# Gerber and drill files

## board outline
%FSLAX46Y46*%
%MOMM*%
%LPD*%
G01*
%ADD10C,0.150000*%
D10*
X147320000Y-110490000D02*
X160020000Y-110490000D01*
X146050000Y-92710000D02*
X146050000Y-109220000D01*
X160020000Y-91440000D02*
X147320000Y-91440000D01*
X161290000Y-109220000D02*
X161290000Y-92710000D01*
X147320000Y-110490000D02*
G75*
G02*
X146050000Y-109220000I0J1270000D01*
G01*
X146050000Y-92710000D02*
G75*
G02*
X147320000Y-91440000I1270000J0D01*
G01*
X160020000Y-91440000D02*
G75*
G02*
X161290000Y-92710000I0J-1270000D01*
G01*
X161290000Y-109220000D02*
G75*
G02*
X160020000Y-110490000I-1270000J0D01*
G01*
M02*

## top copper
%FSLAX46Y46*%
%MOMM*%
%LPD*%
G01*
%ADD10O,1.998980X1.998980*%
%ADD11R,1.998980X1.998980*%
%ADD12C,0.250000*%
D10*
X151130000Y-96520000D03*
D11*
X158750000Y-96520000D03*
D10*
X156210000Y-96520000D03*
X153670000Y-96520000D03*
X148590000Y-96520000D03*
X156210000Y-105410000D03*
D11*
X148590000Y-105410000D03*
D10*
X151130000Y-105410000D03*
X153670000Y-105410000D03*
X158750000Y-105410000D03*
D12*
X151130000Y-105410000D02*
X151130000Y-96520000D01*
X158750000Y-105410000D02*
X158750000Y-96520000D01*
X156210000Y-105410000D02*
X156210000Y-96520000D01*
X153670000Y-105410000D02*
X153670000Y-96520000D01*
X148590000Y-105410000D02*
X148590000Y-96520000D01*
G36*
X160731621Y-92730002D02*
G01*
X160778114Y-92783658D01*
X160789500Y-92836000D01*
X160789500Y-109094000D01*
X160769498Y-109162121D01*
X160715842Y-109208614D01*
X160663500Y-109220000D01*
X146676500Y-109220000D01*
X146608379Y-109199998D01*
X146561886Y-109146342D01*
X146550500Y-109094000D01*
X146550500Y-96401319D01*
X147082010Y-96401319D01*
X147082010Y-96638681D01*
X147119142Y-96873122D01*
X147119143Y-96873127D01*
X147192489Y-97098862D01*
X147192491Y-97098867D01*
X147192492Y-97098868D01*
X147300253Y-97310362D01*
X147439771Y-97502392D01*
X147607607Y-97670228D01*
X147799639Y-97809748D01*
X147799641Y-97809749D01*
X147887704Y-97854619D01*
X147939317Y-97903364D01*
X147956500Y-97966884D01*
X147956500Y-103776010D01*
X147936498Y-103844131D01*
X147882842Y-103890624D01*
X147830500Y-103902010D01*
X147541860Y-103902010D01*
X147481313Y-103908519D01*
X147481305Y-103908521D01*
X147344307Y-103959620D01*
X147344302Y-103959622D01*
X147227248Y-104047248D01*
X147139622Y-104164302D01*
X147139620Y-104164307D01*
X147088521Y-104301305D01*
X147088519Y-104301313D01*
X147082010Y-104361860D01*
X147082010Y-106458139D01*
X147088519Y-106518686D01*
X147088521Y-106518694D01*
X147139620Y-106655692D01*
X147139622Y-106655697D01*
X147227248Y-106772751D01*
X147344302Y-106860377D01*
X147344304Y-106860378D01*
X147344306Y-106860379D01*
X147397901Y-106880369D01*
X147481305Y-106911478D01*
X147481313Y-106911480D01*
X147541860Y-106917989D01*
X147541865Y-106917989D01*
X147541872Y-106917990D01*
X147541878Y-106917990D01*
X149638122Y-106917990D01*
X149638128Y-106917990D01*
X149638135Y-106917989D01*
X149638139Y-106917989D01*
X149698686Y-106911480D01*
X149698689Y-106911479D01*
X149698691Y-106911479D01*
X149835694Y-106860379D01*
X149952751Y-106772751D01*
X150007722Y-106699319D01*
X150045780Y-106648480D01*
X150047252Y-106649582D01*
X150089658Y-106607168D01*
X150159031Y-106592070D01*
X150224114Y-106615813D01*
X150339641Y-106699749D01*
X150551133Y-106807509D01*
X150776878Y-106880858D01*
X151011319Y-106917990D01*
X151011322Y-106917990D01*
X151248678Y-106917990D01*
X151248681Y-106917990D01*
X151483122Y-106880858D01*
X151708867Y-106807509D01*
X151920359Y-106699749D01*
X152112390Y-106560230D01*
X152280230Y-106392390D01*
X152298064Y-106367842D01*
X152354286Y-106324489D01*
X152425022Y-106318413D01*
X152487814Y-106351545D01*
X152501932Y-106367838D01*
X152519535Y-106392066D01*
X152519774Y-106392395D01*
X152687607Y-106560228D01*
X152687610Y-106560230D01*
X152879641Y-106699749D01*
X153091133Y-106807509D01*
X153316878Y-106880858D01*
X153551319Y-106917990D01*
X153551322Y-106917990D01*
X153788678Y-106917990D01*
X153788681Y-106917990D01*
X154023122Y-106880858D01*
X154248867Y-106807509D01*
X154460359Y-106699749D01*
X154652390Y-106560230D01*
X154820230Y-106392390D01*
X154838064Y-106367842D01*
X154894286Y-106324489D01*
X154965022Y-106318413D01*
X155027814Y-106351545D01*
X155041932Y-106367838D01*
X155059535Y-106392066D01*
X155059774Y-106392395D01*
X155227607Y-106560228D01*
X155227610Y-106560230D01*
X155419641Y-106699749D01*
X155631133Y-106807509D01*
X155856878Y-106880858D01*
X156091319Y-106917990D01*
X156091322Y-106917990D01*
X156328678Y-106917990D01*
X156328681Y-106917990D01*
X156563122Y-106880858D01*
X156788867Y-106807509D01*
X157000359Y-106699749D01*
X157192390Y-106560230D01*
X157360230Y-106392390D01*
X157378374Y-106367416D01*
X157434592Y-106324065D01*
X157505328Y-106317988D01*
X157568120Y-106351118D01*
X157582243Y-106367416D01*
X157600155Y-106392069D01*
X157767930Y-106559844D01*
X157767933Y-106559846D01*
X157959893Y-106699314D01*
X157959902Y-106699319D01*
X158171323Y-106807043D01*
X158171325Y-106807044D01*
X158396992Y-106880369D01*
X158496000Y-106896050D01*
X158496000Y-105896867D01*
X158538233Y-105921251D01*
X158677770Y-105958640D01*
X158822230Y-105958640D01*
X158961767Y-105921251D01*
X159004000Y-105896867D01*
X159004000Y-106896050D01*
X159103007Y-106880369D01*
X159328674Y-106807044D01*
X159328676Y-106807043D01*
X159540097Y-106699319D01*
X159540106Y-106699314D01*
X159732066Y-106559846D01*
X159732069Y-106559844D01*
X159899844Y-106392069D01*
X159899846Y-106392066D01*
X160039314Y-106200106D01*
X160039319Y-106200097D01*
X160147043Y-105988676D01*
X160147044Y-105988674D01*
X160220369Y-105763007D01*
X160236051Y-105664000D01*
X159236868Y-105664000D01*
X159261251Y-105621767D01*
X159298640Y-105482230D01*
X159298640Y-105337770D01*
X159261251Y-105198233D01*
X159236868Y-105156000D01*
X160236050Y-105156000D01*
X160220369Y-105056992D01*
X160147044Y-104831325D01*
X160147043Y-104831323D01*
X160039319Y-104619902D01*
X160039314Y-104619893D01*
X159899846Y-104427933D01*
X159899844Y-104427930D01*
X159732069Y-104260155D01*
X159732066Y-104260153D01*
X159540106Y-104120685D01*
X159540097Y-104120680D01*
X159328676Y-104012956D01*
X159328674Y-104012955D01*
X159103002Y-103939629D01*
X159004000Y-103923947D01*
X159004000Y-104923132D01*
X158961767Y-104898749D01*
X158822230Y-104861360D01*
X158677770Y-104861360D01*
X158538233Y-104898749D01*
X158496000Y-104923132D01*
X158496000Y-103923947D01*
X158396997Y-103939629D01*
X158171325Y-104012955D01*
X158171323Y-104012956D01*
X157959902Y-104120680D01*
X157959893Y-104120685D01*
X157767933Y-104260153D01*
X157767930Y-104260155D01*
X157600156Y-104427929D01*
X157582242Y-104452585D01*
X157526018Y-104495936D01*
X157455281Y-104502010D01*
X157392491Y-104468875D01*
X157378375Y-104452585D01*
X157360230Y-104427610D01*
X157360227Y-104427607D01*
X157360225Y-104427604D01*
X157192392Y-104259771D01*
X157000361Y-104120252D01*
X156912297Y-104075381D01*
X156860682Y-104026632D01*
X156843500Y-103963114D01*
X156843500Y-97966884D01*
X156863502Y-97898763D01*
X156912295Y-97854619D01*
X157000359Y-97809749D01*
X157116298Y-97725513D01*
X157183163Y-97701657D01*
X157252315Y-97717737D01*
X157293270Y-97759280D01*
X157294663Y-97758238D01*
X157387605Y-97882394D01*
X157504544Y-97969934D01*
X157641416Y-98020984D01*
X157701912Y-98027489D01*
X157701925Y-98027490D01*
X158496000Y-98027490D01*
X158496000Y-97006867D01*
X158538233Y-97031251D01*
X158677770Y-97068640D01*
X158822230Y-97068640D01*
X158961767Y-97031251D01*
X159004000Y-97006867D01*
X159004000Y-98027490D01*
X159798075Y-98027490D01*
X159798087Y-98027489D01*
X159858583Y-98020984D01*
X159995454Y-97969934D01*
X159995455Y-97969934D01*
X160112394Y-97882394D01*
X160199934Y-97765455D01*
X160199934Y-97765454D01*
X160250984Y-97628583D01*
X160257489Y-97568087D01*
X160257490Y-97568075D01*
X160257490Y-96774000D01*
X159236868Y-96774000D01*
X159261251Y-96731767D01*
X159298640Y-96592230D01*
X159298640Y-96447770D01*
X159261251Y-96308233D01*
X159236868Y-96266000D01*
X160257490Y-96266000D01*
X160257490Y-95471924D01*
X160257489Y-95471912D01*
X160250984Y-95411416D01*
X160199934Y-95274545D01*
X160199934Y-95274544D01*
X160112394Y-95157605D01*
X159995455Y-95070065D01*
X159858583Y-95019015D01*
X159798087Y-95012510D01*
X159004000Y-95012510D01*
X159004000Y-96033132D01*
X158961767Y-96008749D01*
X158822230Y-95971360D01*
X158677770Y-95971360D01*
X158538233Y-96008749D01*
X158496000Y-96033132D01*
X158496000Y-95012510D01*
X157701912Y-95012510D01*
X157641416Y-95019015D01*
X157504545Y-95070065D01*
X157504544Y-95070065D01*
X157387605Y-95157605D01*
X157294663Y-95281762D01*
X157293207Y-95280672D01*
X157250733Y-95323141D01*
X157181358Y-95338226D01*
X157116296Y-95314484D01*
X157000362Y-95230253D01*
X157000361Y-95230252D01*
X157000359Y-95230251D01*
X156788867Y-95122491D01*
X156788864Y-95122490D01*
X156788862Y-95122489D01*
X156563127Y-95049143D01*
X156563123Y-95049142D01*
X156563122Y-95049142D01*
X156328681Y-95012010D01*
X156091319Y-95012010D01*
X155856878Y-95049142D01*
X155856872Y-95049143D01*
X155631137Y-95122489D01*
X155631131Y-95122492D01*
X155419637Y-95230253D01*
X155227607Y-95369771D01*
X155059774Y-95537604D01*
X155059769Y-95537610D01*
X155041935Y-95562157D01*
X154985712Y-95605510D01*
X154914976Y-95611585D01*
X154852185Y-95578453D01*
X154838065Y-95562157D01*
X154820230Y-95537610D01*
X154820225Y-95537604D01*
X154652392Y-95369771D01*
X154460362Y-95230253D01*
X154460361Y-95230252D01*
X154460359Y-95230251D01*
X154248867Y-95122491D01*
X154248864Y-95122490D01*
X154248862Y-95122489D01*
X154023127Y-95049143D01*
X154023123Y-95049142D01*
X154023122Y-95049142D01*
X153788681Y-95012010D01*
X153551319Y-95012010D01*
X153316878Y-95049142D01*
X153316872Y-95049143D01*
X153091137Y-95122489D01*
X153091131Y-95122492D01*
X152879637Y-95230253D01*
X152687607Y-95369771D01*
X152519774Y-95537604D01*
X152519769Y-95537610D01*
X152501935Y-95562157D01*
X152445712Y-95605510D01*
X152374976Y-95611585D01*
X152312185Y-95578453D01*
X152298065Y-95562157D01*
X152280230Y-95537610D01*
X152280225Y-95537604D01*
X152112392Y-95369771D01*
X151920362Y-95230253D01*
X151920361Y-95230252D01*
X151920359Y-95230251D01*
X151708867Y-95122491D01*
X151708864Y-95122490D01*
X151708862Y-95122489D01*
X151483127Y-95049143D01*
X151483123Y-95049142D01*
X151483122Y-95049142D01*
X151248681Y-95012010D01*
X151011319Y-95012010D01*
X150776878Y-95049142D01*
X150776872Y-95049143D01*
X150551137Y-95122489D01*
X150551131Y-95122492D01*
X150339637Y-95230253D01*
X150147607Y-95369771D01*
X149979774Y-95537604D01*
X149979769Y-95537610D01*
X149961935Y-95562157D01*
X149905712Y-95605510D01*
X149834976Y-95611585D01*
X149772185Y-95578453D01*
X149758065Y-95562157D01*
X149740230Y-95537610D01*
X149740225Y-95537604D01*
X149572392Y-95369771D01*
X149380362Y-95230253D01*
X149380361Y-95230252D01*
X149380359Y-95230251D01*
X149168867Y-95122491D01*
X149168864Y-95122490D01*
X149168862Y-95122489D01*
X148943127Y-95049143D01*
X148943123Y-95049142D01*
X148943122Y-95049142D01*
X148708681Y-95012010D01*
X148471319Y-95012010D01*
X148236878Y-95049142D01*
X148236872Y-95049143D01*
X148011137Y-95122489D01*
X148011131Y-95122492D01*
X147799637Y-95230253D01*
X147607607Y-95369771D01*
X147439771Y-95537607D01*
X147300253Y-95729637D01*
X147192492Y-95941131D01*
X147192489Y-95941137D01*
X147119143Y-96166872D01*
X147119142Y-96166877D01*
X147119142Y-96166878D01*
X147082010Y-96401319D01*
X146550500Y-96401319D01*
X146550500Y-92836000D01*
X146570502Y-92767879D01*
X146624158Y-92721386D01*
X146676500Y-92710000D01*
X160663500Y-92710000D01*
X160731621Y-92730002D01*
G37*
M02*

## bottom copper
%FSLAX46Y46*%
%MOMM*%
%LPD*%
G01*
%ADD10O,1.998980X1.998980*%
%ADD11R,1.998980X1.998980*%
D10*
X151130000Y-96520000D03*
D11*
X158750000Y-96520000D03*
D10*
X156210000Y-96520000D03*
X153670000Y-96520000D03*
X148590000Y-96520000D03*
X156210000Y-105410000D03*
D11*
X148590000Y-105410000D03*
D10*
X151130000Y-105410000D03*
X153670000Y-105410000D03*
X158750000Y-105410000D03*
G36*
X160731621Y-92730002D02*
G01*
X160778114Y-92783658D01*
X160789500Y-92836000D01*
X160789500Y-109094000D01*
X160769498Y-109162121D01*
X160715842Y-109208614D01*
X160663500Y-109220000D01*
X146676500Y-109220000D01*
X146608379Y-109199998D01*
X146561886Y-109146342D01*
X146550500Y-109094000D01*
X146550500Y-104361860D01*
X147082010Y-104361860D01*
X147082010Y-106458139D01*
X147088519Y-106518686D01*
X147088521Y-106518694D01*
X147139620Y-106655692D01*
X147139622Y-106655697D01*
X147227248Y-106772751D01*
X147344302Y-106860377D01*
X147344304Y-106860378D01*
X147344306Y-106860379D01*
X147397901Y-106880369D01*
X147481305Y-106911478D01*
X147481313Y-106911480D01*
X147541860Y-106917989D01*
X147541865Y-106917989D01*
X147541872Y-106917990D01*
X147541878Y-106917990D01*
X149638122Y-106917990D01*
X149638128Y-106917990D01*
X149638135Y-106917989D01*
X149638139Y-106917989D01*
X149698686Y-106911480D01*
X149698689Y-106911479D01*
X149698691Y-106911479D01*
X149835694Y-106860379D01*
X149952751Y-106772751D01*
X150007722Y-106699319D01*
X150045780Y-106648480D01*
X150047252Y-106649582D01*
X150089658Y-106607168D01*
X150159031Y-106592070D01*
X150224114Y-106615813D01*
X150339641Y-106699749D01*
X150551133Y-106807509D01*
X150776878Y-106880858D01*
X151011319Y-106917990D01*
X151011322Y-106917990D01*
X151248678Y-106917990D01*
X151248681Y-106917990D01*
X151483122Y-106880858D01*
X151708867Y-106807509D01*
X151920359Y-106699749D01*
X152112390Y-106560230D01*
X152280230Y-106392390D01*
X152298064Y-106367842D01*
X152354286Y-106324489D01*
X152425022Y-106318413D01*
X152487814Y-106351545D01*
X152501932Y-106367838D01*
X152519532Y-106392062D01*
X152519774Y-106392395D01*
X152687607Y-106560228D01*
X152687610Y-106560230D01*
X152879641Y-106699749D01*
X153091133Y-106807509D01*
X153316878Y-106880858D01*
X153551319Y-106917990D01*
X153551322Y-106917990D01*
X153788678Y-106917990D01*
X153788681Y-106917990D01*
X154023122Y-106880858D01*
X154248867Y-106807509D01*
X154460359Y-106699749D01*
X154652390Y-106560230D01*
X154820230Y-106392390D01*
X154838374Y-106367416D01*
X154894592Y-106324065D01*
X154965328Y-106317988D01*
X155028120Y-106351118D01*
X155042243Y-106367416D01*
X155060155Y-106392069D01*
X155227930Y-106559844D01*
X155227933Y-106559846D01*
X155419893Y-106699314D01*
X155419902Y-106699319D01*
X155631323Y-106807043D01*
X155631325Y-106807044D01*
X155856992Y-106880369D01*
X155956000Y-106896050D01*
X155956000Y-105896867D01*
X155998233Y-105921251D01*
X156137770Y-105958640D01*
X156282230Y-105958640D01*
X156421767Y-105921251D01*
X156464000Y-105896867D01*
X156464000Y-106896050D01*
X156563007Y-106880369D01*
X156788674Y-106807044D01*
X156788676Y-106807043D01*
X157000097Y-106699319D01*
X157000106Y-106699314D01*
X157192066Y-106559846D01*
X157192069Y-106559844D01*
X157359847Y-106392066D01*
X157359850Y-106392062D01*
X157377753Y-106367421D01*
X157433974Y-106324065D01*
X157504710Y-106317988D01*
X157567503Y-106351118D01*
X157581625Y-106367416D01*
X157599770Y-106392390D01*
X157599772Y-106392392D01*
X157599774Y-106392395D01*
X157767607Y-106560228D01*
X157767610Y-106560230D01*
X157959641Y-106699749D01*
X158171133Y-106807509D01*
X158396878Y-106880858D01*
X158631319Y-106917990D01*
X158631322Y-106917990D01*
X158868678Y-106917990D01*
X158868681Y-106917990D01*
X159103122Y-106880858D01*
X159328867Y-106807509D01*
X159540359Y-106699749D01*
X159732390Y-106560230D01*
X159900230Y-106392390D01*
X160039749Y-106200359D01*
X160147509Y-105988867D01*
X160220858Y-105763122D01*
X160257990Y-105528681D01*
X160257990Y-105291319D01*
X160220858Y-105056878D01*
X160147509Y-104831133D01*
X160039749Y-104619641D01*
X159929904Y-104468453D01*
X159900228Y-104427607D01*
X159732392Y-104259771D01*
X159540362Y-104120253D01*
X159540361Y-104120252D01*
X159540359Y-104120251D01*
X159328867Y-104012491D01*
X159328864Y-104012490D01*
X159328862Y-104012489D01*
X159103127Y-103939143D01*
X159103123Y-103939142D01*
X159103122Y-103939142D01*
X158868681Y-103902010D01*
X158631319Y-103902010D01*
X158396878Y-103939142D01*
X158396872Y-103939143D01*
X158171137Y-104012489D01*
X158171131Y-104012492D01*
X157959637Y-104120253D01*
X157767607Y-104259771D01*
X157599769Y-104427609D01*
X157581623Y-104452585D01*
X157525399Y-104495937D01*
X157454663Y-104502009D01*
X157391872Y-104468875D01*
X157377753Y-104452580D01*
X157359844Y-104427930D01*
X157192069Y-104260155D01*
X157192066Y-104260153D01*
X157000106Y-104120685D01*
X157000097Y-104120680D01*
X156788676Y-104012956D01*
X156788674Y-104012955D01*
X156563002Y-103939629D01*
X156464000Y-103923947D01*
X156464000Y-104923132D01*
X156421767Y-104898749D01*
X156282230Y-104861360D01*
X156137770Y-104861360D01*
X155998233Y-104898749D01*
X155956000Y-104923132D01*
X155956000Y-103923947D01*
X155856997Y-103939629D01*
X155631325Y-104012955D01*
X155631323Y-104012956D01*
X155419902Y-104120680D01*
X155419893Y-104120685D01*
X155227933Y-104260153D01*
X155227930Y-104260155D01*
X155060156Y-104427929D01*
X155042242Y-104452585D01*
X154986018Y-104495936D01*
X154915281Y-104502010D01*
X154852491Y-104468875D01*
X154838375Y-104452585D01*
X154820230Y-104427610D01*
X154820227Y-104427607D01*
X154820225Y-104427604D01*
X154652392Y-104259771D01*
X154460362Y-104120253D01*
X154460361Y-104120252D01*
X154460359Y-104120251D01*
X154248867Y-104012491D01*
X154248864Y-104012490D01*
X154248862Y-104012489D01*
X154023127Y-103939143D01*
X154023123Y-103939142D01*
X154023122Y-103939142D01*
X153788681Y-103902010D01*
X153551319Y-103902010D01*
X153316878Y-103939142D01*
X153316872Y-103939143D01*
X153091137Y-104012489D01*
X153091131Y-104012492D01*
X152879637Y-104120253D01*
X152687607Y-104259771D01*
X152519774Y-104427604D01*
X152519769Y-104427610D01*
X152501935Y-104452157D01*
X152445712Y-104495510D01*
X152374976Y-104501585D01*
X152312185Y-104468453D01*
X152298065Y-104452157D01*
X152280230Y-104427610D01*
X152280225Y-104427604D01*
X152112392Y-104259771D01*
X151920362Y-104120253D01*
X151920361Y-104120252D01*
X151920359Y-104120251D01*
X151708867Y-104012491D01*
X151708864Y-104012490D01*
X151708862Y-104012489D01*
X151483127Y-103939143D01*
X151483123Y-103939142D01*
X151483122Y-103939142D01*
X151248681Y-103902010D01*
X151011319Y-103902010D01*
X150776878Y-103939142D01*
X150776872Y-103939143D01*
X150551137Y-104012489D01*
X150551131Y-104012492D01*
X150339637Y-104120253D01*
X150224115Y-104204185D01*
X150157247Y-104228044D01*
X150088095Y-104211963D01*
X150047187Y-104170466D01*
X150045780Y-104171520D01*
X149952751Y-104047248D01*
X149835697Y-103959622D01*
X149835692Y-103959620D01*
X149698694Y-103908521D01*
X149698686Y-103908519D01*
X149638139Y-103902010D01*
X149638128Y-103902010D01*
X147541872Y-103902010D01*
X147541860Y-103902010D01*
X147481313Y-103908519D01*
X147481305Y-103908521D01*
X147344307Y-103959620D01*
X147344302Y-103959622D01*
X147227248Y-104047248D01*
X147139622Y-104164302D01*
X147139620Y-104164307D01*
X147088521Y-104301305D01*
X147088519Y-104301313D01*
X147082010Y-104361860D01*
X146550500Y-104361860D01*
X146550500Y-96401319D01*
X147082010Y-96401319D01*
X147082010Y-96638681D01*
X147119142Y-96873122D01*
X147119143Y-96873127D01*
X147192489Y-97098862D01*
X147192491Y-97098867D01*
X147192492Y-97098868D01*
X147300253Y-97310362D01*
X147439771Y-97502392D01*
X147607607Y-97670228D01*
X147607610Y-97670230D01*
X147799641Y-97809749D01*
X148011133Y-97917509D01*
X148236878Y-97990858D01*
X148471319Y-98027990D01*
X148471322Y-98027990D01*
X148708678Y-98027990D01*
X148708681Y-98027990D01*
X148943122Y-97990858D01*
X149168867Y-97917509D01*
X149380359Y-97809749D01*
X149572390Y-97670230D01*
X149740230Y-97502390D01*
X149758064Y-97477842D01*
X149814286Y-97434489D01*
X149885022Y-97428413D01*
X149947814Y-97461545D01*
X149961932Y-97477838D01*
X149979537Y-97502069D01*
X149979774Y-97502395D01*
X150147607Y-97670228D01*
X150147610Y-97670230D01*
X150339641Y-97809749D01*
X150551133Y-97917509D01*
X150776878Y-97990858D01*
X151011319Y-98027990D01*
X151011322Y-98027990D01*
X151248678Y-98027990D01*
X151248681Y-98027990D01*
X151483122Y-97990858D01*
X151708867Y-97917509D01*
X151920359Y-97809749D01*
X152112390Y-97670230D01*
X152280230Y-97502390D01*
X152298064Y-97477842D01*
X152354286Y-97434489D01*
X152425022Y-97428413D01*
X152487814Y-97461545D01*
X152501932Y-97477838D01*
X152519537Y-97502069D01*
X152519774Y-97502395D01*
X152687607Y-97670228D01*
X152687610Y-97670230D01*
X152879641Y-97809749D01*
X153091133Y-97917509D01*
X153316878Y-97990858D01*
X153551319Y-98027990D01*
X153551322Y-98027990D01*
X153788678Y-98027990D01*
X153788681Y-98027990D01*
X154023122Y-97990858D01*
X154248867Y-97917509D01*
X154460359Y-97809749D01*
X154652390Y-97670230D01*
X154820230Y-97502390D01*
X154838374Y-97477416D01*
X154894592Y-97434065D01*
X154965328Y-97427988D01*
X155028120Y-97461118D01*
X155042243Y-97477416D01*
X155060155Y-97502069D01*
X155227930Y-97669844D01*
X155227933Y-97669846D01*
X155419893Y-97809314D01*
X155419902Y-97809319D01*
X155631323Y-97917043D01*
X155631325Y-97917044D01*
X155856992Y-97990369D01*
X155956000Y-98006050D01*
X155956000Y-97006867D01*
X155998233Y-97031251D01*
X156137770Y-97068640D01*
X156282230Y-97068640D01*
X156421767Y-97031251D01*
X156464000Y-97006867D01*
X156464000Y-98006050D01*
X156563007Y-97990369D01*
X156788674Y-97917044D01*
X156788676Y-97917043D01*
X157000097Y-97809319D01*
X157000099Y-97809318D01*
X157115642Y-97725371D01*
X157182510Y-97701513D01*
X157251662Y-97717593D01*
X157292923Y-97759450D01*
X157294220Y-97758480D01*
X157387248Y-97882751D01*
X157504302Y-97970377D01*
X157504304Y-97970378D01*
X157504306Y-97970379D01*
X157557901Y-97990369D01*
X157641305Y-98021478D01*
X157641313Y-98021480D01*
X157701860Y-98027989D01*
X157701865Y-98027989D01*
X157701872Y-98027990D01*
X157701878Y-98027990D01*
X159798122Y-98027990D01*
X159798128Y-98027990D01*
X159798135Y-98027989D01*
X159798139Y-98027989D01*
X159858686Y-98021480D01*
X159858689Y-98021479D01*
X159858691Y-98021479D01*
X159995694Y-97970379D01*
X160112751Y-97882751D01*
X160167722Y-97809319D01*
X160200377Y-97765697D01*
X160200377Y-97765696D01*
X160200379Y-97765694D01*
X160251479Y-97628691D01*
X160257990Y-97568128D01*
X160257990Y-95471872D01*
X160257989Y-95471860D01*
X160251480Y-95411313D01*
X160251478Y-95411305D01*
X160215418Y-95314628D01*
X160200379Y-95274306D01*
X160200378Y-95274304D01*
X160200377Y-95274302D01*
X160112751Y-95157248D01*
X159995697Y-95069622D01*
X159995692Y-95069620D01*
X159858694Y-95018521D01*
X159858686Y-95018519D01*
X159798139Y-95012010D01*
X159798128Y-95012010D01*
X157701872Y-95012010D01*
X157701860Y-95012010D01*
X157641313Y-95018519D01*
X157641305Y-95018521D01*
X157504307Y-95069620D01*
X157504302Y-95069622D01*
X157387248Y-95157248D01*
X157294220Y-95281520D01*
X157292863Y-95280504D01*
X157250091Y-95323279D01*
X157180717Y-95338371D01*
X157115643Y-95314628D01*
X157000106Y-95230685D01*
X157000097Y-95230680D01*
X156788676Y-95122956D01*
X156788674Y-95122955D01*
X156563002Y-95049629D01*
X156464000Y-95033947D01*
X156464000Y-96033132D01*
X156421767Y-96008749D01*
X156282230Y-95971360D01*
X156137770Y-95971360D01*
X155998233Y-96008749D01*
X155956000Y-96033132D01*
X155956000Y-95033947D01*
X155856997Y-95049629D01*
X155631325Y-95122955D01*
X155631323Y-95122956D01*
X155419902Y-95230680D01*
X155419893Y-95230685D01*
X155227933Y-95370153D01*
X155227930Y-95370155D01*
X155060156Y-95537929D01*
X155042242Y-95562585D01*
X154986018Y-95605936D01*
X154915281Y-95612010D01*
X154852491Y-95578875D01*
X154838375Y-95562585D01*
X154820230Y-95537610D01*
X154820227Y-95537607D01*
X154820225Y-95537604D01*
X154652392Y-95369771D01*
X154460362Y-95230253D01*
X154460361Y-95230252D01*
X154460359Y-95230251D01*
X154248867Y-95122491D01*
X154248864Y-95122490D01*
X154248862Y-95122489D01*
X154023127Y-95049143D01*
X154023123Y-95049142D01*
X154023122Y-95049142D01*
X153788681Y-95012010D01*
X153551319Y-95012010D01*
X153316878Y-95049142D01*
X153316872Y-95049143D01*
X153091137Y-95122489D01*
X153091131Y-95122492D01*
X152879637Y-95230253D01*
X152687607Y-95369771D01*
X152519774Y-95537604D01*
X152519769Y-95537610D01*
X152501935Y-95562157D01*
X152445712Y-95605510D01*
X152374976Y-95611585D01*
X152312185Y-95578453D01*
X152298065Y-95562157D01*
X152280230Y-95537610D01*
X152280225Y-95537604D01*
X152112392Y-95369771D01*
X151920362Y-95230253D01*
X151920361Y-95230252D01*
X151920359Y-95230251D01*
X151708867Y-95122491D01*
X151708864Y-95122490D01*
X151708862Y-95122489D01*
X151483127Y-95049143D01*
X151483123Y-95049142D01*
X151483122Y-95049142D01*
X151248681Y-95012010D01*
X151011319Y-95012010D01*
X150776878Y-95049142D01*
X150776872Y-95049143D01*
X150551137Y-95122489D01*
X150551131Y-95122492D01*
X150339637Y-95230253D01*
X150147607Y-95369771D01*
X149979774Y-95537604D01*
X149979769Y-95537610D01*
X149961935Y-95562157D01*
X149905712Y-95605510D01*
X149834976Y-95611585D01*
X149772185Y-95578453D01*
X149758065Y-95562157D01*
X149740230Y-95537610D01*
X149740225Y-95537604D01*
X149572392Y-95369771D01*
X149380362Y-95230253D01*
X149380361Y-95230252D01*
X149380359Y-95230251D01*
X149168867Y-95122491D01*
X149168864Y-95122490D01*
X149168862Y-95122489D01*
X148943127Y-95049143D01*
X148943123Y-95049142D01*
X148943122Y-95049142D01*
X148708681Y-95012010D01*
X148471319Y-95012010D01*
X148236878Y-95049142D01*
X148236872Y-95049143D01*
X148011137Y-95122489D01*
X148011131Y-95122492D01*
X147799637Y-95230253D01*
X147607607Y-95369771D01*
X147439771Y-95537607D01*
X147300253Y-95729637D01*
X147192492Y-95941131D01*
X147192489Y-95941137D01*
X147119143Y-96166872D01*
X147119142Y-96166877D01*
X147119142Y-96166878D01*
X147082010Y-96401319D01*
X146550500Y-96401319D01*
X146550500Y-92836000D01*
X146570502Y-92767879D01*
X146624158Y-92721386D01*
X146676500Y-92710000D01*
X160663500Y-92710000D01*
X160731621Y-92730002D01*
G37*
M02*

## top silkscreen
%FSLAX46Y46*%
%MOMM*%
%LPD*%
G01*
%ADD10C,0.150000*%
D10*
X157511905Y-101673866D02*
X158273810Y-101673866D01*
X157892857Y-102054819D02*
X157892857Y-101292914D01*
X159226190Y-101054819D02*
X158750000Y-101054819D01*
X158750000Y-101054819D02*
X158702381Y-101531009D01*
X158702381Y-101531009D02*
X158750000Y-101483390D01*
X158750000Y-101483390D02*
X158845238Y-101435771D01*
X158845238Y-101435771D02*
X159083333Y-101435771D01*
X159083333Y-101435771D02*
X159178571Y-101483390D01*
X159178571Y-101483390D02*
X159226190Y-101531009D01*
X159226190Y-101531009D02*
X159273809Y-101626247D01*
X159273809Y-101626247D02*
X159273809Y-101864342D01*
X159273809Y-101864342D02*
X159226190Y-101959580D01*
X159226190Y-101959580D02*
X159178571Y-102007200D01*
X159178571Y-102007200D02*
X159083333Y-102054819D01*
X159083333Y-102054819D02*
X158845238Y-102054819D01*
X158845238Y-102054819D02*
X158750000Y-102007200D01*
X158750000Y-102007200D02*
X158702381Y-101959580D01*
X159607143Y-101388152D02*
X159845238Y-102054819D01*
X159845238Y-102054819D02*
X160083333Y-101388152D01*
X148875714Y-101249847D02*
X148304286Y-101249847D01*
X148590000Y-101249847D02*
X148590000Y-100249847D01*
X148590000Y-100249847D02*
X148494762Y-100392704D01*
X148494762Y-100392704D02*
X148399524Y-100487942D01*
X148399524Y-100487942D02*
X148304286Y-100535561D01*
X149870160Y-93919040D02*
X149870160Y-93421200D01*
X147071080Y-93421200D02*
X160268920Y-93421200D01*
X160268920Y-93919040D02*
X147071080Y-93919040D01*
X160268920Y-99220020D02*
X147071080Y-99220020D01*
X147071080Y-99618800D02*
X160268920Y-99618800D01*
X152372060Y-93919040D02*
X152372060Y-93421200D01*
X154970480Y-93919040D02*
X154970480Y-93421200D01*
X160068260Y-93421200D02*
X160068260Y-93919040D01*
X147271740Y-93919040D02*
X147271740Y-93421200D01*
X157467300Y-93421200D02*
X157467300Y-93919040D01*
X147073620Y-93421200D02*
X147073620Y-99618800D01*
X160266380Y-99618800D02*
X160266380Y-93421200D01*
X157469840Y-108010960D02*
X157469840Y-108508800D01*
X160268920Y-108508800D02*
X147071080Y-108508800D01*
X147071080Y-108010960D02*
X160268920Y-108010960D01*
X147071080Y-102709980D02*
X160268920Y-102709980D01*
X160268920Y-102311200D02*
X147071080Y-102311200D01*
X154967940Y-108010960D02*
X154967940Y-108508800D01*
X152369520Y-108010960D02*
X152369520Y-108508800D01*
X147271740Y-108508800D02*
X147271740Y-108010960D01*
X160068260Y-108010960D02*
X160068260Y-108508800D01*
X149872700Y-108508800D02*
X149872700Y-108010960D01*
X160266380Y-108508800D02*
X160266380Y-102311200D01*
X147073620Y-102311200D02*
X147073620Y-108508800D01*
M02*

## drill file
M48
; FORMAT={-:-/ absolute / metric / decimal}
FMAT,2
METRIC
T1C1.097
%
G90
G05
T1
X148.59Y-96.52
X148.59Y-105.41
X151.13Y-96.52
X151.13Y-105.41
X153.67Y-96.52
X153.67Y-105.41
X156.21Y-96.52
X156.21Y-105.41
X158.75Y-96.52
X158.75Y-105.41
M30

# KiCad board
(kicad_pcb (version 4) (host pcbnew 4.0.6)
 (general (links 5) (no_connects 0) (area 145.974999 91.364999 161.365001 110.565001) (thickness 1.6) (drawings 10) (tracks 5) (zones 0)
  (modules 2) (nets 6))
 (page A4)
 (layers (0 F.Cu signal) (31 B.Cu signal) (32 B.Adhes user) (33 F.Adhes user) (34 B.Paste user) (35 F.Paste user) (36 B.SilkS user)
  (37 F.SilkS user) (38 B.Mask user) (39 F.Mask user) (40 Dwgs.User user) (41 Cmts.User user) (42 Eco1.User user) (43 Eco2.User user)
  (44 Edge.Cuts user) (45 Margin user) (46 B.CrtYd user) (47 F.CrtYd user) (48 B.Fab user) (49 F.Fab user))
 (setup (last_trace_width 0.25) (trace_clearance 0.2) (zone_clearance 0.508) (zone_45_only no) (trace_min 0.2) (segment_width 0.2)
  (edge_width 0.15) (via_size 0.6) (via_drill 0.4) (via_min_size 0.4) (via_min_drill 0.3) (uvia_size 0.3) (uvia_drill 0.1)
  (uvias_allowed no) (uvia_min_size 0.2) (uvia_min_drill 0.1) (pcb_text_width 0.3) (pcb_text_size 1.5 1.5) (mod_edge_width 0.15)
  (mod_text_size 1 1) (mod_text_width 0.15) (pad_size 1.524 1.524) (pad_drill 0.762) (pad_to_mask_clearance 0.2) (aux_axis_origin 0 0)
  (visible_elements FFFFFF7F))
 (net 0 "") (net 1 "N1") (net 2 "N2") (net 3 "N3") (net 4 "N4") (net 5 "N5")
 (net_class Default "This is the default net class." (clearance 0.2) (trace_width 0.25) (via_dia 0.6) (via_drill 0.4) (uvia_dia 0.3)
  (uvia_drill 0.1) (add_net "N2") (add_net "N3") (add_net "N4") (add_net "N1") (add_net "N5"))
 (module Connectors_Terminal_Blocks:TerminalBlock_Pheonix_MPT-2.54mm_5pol (layer F.Cu) (at 158.75 96.52 180)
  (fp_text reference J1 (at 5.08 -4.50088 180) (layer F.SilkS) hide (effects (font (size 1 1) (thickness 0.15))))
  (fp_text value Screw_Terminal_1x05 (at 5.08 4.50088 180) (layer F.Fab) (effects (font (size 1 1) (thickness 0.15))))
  (fp_line (start 8.87984 2.60096) (end 8.87984 3.0988) (layer F.SilkS) (width 0.15))
  (fp_line (start 11.67892 3.0988) (end -1.51892 3.0988) (layer F.SilkS) (width 0.15))
  (fp_line (start -1.51892 2.60096) (end 11.67892 2.60096) (layer F.SilkS) (width 0.15))
  (fp_line (start -1.51892 -2.70002) (end 11.67892 -2.70002) (layer F.SilkS) (width 0.15))
  (fp_line (start 11.67892 -3.0988) (end -1.51892 -3.0988) (layer F.SilkS) (width 0.15))
  (fp_line (start 6.37794 2.60096) (end 6.37794 3.0988) (layer F.SilkS) (width 0.15))
  (fp_line (start 3.77952 2.60096) (end 3.77952 3.0988) (layer F.SilkS) (width 0.15))
  (fp_line (start -1.31826 3.0988) (end -1.31826 2.60096) (layer F.SilkS) (width 0.15))
  (fp_line (start 11.47826 2.60096) (end 11.47826 3.0988) (layer F.SilkS) (width 0.15))
  (fp_line (start 1.2827 3.0988) (end 1.2827 2.60096) (layer F.SilkS) (width 0.15))
  (fp_line (start 11.67638 3.0988) (end 11.67638 -3.0988) (layer F.SilkS) (width 0.15))
  (fp_line (start -1.51638 -3.0988) (end -1.51638 3.0988) (layer F.SilkS) (width 0.15))
  (pad 4 thru_hole oval (at 7.62 0) (size 1.99898 1.99898) (drill 1.09728) (layers *.Cu *.Mask) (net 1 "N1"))
  (pad 1 thru_hole rect (at 0 0) (size 1.99898 1.99898) (drill 1.09728) (layers *.Cu *.Mask) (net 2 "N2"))
  (pad 2 thru_hole oval (at 2.54 0) (size 1.99898 1.99898) (drill 1.09728) (layers *.Cu *.Mask) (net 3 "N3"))
  (pad 3 thru_hole oval (at 5.08 0) (size 1.99898 1.99898) (drill 1.09728) (layers *.Cu *.Mask) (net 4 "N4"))
  (pad 5 thru_hole oval (at 10.16 0) (size 1.99898 1.99898) (drill 1.09728) (layers *.Cu *.Mask) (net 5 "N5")))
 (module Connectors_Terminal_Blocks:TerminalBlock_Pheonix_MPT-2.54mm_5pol (layer F.Cu) (at 148.59 105.41)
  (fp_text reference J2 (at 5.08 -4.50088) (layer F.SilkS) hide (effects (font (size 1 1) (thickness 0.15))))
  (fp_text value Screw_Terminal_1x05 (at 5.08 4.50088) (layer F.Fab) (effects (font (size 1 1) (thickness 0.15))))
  (fp_line (start 8.87984 2.60096) (end 8.87984 3.0988) (layer F.SilkS) (width 0.15))
  (fp_line (start 11.67892 3.0988) (end -1.51892 3.0988) (layer F.SilkS) (width 0.15))
  (fp_line (start -1.51892 2.60096) (end 11.67892 2.60096) (layer F.SilkS) (width 0.15))
  (fp_line (start -1.51892 -2.70002) (end 11.67892 -2.70002) (layer F.SilkS) (width 0.15))
  (fp_line (start 11.67892 -3.0988) (end -1.51892 -3.0988) (layer F.SilkS) (width 0.15))
  (fp_line (start 6.37794 2.60096) (end 6.37794 3.0988) (layer F.SilkS) (width 0.15))
  (fp_line (start 3.77952 2.60096) (end 3.77952 3.0988) (layer F.SilkS) (width 0.15))
  (fp_line (start -1.31826 3.0988) (end -1.31826 2.60096) (layer F.SilkS) (width 0.15))
  (fp_line (start 11.47826 2.60096) (end 11.47826 3.0988) (layer F.SilkS) (width 0.15))
  (fp_line (start 1.2827 3.0988) (end 1.2827 2.60096) (layer F.SilkS) (width 0.15))
  (fp_line (start 11.67638 3.0988) (end 11.67638 -3.0988) (layer F.SilkS) (width 0.15))
  (fp_line (start -1.51638 -3.0988) (end -1.51638 3.0988) (layer F.SilkS) (width 0.15))
  (pad 4 thru_hole oval (at 7.62 0 180) (size 1.99898 1.99898) (drill 1.09728) (layers *.Cu *.Mask) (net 3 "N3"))
  (pad 1 thru_hole rect (at 0 0 180) (size 1.99898 1.99898) (drill 1.09728) (layers *.Cu *.Mask) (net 5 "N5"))
  (pad 2 thru_hole oval (at 2.54 0 180) (size 1.99898 1.99898) (drill 1.09728) (layers *.Cu *.Mask) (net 1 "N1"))
  (pad 3 thru_hole oval (at 5.08 0 180) (size 1.99898 1.99898) (drill 1.09728) (layers *.Cu *.Mask) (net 4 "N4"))
  (pad 5 thru_hole oval (at 10.16 0 180) (size 1.99898 1.99898) (drill 1.09728) (layers *.Cu *.Mask) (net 2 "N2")))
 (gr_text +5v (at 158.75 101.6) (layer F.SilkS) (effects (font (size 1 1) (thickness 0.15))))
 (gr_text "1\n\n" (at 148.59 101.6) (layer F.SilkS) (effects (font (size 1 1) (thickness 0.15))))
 (gr_line (start 147.32 110.49) (end 160.02 110.49) (angle 90) (layer Edge.Cuts) (width 0.15))
 (gr_line (start 146.05 92.71) (end 146.05 109.22) (angle 90) (layer Edge.Cuts) (width 0.15))
 (gr_line (start 160.02 91.44) (end 147.32 91.44) (angle 90) (layer Edge.Cuts) (width 0.15))
 (gr_line (start 161.29 109.22) (end 161.29 92.71) (angle 90) (layer Edge.Cuts) (width 0.15))
 (gr_arc (start 147.32 109.22) (end 147.32 110.49) (angle 90) (layer Edge.Cuts) (width 0.15))
 (gr_arc (start 147.32 92.71) (end 146.05 92.71) (angle 90) (layer Edge.Cuts) (width 0.15))
 (gr_arc (start 160.02 92.71) (end 160.02 91.44) (angle 90) (layer Edge.Cuts) (width 0.15))
 (gr_arc (start 160.02 109.22) (end 161.29 109.22) (angle 90) (layer Edge.Cuts) (width 0.15))
 (segment (start 151.13 105.41) (end 151.13 96.52) (width 0.25) (layer F.Cu) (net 1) (status C00000))
 (segment (start 158.75 105.41) (end 158.75 96.52) (width 0.25) (layer F.Cu) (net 2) (status C00000))
 (segment (start 156.21 105.41) (end 156.21 96.52) (width 0.25) (layer F.Cu) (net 3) (status C00000))
 (segment (start 153.67 105.41) (end 153.67 96.52) (width 0.25) (layer F.Cu) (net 4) (status C00000))
 (segment (start 148.59 105.41) (end 148.59 96.52) (width 0.25) (layer F.Cu) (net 5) (status C00000))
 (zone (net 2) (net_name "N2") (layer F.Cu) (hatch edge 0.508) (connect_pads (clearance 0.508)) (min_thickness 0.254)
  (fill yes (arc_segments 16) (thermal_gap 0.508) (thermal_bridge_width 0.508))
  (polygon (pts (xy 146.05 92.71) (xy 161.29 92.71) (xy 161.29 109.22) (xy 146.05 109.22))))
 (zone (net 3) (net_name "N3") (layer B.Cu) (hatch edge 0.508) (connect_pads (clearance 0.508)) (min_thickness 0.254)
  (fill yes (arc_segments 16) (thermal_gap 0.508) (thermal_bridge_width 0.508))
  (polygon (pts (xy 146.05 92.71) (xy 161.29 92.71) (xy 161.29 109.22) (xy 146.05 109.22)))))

